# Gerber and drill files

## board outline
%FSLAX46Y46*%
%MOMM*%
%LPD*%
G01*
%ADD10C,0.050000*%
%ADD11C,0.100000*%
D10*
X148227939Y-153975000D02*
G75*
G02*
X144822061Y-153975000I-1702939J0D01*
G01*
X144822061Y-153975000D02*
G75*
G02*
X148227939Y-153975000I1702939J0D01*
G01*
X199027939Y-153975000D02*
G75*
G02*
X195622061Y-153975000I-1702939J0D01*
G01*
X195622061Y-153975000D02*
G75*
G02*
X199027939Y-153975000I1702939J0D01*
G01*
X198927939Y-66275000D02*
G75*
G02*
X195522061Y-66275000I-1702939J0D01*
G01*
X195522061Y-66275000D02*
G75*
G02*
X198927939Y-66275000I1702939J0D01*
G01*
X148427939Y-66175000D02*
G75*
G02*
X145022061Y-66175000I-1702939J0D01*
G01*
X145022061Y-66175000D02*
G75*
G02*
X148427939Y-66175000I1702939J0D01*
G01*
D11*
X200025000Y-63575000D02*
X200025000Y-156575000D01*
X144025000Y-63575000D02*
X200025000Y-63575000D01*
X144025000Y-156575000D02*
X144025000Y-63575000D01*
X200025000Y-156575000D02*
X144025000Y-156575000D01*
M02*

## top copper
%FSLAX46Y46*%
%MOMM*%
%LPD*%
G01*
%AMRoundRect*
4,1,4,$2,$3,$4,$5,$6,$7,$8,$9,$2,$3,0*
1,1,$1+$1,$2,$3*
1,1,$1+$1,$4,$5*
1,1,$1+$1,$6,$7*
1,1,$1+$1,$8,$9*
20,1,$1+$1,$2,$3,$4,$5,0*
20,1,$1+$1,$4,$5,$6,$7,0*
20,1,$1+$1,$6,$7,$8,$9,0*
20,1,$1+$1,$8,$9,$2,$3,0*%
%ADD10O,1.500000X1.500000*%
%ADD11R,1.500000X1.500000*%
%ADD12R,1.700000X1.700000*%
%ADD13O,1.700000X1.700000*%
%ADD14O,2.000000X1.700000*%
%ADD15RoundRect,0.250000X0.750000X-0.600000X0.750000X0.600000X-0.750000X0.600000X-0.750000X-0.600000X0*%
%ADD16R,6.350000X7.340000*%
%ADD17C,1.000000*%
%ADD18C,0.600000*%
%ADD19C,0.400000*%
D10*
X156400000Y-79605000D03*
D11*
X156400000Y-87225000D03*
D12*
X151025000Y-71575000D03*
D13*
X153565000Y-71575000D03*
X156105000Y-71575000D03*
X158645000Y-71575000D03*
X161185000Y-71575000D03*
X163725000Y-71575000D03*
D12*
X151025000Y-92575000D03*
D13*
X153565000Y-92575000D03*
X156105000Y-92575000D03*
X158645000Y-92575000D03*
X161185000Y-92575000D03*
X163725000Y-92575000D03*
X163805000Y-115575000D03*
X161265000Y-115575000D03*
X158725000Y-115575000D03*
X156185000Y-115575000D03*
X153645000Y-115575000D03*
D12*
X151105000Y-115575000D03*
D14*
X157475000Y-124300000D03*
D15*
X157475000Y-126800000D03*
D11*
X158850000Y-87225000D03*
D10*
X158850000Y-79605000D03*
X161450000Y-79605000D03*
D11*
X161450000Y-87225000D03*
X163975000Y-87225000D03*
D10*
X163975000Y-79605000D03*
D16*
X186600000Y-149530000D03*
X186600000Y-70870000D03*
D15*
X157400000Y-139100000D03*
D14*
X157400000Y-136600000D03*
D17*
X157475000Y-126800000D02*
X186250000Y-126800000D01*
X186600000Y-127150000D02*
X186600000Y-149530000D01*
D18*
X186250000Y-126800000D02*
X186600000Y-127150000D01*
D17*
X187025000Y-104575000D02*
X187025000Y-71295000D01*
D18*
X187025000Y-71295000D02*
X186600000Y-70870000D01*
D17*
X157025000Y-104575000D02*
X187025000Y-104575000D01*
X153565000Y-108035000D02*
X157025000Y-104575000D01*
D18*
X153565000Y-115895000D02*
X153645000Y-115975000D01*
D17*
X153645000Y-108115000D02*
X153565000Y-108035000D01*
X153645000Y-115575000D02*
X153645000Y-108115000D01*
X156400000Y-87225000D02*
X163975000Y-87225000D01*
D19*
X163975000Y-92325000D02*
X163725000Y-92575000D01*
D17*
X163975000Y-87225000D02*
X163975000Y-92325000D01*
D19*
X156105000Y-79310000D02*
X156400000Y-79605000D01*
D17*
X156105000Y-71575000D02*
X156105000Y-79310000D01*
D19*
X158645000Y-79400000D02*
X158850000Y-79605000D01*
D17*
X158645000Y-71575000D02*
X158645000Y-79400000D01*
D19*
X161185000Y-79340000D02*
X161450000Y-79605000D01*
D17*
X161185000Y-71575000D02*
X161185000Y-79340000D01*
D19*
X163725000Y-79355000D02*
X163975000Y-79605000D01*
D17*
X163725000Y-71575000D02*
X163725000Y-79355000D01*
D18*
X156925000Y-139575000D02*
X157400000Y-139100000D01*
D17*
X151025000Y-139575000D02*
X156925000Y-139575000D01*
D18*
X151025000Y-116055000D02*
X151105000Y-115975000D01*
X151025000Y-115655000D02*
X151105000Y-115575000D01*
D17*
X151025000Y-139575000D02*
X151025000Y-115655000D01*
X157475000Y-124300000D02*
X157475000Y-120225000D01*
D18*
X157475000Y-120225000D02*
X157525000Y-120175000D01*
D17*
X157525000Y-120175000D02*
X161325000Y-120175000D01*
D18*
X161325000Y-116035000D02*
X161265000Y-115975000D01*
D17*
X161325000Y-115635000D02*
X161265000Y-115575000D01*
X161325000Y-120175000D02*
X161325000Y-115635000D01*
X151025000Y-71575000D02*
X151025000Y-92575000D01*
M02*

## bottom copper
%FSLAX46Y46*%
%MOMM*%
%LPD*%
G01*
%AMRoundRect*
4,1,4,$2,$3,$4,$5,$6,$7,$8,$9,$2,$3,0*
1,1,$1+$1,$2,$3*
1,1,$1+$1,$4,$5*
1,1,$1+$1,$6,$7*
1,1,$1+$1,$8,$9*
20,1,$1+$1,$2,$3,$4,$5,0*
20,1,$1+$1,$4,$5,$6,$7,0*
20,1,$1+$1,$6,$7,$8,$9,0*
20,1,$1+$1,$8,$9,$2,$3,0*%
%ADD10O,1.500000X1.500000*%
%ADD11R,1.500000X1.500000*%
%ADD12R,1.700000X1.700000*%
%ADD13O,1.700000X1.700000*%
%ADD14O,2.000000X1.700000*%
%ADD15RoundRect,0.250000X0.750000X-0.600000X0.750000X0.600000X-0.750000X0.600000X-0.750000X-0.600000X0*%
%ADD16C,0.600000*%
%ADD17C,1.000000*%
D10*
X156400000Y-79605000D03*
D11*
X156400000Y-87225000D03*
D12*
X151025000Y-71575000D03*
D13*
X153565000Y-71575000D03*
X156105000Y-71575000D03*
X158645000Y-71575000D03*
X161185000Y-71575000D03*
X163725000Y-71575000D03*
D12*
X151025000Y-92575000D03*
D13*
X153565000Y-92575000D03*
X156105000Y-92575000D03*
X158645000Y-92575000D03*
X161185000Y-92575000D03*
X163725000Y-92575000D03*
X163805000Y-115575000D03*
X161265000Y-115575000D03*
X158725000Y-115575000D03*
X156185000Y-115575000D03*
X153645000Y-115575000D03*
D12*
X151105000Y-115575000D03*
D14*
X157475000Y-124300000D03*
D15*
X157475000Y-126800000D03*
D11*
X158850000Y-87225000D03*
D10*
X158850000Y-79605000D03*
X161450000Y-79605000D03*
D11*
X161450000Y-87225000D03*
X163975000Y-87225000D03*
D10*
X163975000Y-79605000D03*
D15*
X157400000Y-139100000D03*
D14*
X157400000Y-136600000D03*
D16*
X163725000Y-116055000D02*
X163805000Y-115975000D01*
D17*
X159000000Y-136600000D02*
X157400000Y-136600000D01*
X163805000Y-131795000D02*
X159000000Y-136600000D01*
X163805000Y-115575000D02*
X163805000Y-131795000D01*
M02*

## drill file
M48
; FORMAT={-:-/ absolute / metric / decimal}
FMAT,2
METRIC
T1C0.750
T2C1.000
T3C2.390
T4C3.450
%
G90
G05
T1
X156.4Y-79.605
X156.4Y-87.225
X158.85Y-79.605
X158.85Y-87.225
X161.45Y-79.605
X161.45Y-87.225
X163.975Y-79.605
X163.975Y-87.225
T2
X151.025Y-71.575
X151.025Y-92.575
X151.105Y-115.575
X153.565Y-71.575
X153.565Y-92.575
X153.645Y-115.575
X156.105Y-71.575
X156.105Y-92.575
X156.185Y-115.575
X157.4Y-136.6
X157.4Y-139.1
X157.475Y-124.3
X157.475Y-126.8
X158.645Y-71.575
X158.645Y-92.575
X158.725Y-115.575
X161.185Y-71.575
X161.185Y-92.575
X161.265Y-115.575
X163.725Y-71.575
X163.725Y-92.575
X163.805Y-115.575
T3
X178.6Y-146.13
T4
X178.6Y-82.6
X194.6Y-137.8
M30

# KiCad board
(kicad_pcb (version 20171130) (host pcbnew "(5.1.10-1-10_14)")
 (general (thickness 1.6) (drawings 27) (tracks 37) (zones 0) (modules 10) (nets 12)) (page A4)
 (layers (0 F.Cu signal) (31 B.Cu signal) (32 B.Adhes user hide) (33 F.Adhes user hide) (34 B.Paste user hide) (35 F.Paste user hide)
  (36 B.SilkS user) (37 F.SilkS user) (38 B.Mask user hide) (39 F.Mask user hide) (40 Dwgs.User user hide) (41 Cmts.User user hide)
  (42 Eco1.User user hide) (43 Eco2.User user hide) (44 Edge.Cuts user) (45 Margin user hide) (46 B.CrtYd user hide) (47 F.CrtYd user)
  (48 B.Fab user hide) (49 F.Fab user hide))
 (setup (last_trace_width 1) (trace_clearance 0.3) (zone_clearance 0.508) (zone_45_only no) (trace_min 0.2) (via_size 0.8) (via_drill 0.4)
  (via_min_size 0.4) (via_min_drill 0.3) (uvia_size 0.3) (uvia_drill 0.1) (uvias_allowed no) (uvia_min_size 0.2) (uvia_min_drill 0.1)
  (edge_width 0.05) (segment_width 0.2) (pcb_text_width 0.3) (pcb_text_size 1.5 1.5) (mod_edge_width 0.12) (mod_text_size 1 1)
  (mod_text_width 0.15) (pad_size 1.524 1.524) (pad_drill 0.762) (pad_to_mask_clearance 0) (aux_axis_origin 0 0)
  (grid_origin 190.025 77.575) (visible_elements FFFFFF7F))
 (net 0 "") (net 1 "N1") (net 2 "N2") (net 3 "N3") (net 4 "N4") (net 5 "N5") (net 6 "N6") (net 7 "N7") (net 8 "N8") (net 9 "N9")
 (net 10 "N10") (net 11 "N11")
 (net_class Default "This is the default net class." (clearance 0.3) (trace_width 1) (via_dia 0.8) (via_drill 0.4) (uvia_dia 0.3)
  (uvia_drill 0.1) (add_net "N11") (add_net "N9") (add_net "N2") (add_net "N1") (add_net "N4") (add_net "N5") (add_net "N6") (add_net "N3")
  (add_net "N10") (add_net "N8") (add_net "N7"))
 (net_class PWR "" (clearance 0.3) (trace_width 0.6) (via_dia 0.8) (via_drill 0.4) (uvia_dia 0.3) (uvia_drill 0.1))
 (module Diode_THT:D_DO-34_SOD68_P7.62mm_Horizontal (layer F.Cu) (at 156.4 87.225 90)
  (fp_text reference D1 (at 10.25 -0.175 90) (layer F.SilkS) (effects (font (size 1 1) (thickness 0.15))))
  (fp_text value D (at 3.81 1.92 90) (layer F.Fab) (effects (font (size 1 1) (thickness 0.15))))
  (pad 2 thru_hole oval (at 7.62 0 90) (size 1.5 1.5) (drill 0.75) (layers *.Cu *.Mask) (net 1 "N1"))
  (pad 1 thru_hole rect (at 0 0 90) (size 1.5 1.5) (drill 0.75) (layers *.Cu *.Mask) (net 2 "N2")))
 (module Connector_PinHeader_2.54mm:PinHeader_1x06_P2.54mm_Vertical (layer F.Cu) (at 151.025 71.575 90)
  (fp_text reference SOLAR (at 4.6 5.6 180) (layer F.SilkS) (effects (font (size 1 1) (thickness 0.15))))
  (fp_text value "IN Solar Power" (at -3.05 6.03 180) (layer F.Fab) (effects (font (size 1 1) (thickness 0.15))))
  (pad 1 thru_hole rect (at 0 0 90) (size 1.7 1.7) (drill 1) (layers *.Cu *.Mask) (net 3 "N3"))
  (pad 2 thru_hole oval (at 0 2.54 90) (size 1.7 1.7) (drill 1) (layers *.Cu *.Mask))
  (pad 3 thru_hole oval (at 0 5.08 90) (size 1.7 1.7) (drill 1) (layers *.Cu *.Mask) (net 1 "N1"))
  (pad 4 thru_hole oval (at 0 7.62 90) (size 1.7 1.7) (drill 1) (layers *.Cu *.Mask) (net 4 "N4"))
  (pad 5 thru_hole oval (at 0 10.16 90) (size 1.7 1.7) (drill 1) (layers *.Cu *.Mask) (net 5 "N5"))
  (pad 6 thru_hole oval (at 0 12.7 90) (size 1.7 1.7) (drill 1) (layers *.Cu *.Mask) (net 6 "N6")))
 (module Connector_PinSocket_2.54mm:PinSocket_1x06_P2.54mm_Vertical (layer F.Cu) (at 151.025 92.575 90)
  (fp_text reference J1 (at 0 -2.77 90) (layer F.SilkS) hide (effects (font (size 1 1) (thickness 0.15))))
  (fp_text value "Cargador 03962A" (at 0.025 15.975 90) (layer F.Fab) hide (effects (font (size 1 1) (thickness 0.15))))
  (pad 1 thru_hole rect (at 0 0 90) (size 1.7 1.7) (drill 1) (layers *.Cu *.Mask) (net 3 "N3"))
  (pad 2 thru_hole oval (at 0 2.54 90) (size 1.7 1.7) (drill 1) (layers *.Cu *.Mask))
  (pad 3 thru_hole oval (at 0 5.08 90) (size 1.7 1.7) (drill 1) (layers *.Cu *.Mask))
  (pad 4 thru_hole oval (at 0 7.62 90) (size 1.7 1.7) (drill 1) (layers *.Cu *.Mask))
  (pad 5 thru_hole oval (at 0 10.16 90) (size 1.7 1.7) (drill 1) (layers *.Cu *.Mask))
  (pad 6 thru_hole oval (at 0 12.7 90) (size 1.7 1.7) (drill 1) (layers *.Cu *.Mask) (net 2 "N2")))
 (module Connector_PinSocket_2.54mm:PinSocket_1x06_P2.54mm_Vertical (layer F.Cu) (at 151.105 115.575 90)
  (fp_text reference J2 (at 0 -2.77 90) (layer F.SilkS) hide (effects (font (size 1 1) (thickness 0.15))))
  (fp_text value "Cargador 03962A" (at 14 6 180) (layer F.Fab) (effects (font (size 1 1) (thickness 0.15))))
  (pad 6 thru_hole oval (at 0 12.7 90) (size 1.7 1.7) (drill 1) (layers *.Cu *.Mask) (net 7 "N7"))
  (pad 5 thru_hole oval (at 0 10.16 90) (size 1.7 1.7) (drill 1) (layers *.Cu *.Mask) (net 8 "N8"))
  (pad 4 thru_hole oval (at 0 7.62 90) (size 1.7 1.7) (drill 1) (layers *.Cu *.Mask))
  (pad 3 thru_hole oval (at 0 5.08 90) (size 1.7 1.7) (drill 1) (layers *.Cu *.Mask))
  (pad 2 thru_hole oval (at 0 2.54 90) (size 1.7 1.7) (drill 1) (layers *.Cu *.Mask) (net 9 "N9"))
  (pad 1 thru_hole rect (at 0 0 90) (size 1.7 1.7) (drill 1) (layers *.Cu *.Mask) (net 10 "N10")))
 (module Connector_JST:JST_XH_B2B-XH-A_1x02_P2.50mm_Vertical (layer F.Cu) (at 157.475 126.8 90)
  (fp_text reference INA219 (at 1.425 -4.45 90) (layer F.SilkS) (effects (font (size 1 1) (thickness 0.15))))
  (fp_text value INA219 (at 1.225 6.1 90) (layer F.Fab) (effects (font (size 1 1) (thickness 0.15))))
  (pad 2 thru_hole oval (at 2.5 0 90) (size 1.7 2) (drill 1) (layers *.Cu *.Mask) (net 8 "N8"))
  (pad 1 thru_hole roundrect (at 0 0 90) (size 1.7 2) (drill 1) (layers *.Cu *.Mask) (roundrect_rratio 0.147059) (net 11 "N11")))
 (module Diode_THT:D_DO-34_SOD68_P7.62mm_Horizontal (layer F.Cu) (at 158.85 87.225 90)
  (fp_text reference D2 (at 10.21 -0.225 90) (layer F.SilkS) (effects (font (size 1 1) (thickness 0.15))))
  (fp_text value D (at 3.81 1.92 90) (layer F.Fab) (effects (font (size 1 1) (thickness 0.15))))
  (pad 1 thru_hole rect (at 0 0 90) (size 1.5 1.5) (drill 0.75) (layers *.Cu *.Mask) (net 2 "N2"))
  (pad 2 thru_hole oval (at 7.62 0 90) (size 1.5 1.5) (drill 0.75) (layers *.Cu *.Mask) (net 4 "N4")))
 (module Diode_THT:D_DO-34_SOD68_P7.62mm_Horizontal (layer F.Cu) (at 161.45 87.225 90)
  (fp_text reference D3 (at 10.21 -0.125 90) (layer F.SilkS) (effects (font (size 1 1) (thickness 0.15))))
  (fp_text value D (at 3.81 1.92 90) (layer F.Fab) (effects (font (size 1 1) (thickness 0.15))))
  (pad 2 thru_hole oval (at 7.62 0 90) (size 1.5 1.5) (drill 0.75) (layers *.Cu *.Mask) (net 5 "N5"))
  (pad 1 thru_hole rect (at 0 0 90) (size 1.5 1.5) (drill 0.75) (layers *.Cu *.Mask) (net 2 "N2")))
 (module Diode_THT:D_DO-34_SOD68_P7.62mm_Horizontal (layer F.Cu) (at 163.975 87.225 90)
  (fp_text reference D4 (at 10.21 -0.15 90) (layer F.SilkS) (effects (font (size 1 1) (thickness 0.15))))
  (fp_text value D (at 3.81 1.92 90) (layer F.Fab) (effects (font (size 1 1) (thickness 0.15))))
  (pad 1 thru_hole rect (at 0 0 90) (size 1.5 1.5) (drill 0.75) (layers *.Cu *.Mask) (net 2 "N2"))
  (pad 2 thru_hole oval (at 7.62 0 90) (size 1.5 1.5) (drill 0.75) (layers *.Cu *.Mask) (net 6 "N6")))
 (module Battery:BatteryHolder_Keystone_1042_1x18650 (layer F.Cu) (at 186.6 110.2 90)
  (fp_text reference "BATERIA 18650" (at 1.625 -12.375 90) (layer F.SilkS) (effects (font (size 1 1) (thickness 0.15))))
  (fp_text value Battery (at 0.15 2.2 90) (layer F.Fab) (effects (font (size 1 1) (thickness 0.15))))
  (pad 1 smd rect (at -39.33 0 90) (size 7.34 6.35) (layers F.Cu F.Paste F.Mask) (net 11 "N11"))
  (pad 2 smd rect (at 39.33 0 90) (size 7.34 6.35) (layers F.Cu F.Paste F.Mask) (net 9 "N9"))
  (pad "" np_thru_hole circle (at 27.6 -8 90) (size 3.45 3.45) (drill 3.45) (layers *.Cu *.Mask))
  (pad "" np_thru_hole circle (at -27.6 8 90) (size 3.45 3.45) (drill 3.45) (layers *.Cu *.Mask))
  (pad "" np_thru_hole circle (at -35.93 -8 90) (size 2.39 2.39) (drill 2.39) (layers *.Cu *.Mask)))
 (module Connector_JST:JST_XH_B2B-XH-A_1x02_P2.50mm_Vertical (layer F.Cu) (at 157.4 139.1 90)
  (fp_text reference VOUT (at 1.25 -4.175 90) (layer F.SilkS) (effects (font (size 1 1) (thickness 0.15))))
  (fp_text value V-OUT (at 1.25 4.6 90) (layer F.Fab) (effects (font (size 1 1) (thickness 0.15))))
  (pad 1 thru_hole roundrect (at 0 0 90) (size 1.7 2) (drill 1) (layers *.Cu *.Mask) (roundrect_rratio 0.147059) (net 10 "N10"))
  (pad 2 thru_hole oval (at 2.5 0 90) (size 1.7 2) (drill 1) (layers *.Cu *.Mask) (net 7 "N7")))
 (gr_circle (center 146.525 153.975) (end 148.225 153.875) (layer Edge.Cuts) (width 0.05))
 (gr_circle (center 197.325 153.975) (end 199.025 153.875) (layer Edge.Cuts) (width 0.05))
 (gr_circle (center 197.225 66.275) (end 198.925 66.175) (layer Edge.Cuts) (width 0.05))
 (gr_circle (center 146.725 66.175) (end 148.425 66.075) (layer Edge.Cuts) (width 0.05))
 (gr_line (start 200.025 63.575) (end 200.025 156.575) (layer Edge.Cuts) (width 0.1))
 (gr_line (start 144.025 63.575) (end 200.025 63.575) (layer Edge.Cuts) (width 0.1))
 (gr_line (start 144.025 156.575) (end 144.025 63.575) (layer Edge.Cuts) (width 0.1))
 (gr_line (start 200.025 156.575) (end 144.025 156.575) (layer Edge.Cuts) (width 0.1))
 (segment (start 157.475 126.8) (end 186.25 126.8) (width 1) (layer F.Cu) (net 11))
 (segment (start 186.6 127.15) (end 186.6 149.53) (width 1) (layer F.Cu) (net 11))
 (segment (start 186.25 126.8) (end 186.6 127.15) (width 0.6) (layer F.Cu) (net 11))
 (segment (start 187.025 104.575) (end 187.025 71.295) (width 1) (layer F.Cu) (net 9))
 (segment (start 187.025 71.295) (end 186.6 70.87) (width 0.6) (layer F.Cu) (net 9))
 (segment (start 157.025 104.575) (end 187.025 104.575) (width 1) (layer F.Cu) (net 9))
 (segment (start 153.565 108.035) (end 157.025 104.575) (width 1) (layer F.Cu) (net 9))
 (segment (start 153.565 115.895) (end 153.645 115.975) (width 0.6) (layer F.Cu) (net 9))
 (segment (start 153.645 108.115) (end 153.565 108.035) (width 1) (layer F.Cu) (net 9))
 (segment (start 153.645 115.575) (end 153.645 108.115) (width 1) (layer F.Cu) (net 9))
 (segment (start 156.4 87.225) (end 163.975 87.225) (width 1) (layer F.Cu) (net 2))
 (segment (start 163.975 92.325) (end 163.725 92.575) (width 0.4) (layer F.Cu) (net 2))
 (segment (start 163.975 87.225) (end 163.975 92.325) (width 1) (layer F.Cu) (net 2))
 (segment (start 156.105 79.31) (end 156.4 79.605) (width 0.4) (layer F.Cu) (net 1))
 (segment (start 156.105 71.575) (end 156.105 79.31) (width 1) (layer F.Cu) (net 1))
 (segment (start 158.645 79.4) (end 158.85 79.605) (width 0.4) (layer F.Cu) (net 4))
 (segment (start 158.645 71.575) (end 158.645 79.4) (width 1) (layer F.Cu) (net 4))
 (segment (start 161.185 79.34) (end 161.45 79.605) (width 0.4) (layer F.Cu) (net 5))
 (segment (start 161.185 71.575) (end 161.185 79.34) (width 1) (layer F.Cu) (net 5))
 (segment (start 163.725 79.355) (end 163.975 79.605) (width 0.4) (layer F.Cu) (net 6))
 (segment (start 163.725 71.575) (end 163.725 79.355) (width 1) (layer F.Cu) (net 6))
 (segment (start 163.725 116.055) (end 163.805 115.975) (width 0.6) (layer B.Cu) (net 7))
 (segment (start 159 136.6) (end 157.4 136.6) (width 1) (layer B.Cu) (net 7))
 (segment (start 163.805 131.795) (end 159 136.6) (width 1) (layer B.Cu) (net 7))
 (segment (start 163.805 115.575) (end 163.805 131.795) (width 1) (layer B.Cu) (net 7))
 (segment (start 156.925 139.575) (end 157.4 139.1) (width 0.6) (layer F.Cu) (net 10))
 (segment (start 151.025 139.575) (end 156.925 139.575) (width 1) (layer F.Cu) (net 10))
 (segment (start 151.025 116.055) (end 151.105 115.975) (width 0.6) (layer F.Cu) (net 10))
 (segment (start 151.025 115.655) (end 151.105 115.575) (width 0.6) (layer F.Cu) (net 10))
 (segment (start 151.025 139.575) (end 151.025 115.655) (width 1) (layer F.Cu) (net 10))
 (segment (start 157.475 124.3) (end 157.475 120.225) (width 1) (layer F.Cu) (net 8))
 (segment (start 157.475 120.225) (end 157.525 120.175) (width 0.6) (layer F.Cu) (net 8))
 (segment (start 157.525 120.175) (end 161.325 120.175) (width 1) (layer F.Cu) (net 8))
 (segment (start 161.325 116.035) (end 161.265 115.975) (width 0.6) (layer F.Cu) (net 8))
 (segment (start 161.325 115.635) (end 161.265 115.575) (width 1) (layer F.Cu) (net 8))
 (segment (start 161.325 120.175) (end 161.325 115.635) (width 1) (layer F.Cu) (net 8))
 (segment (start 151.025 71.575) (end 151.025 92.575) (width 1) (layer F.Cu) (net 3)))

